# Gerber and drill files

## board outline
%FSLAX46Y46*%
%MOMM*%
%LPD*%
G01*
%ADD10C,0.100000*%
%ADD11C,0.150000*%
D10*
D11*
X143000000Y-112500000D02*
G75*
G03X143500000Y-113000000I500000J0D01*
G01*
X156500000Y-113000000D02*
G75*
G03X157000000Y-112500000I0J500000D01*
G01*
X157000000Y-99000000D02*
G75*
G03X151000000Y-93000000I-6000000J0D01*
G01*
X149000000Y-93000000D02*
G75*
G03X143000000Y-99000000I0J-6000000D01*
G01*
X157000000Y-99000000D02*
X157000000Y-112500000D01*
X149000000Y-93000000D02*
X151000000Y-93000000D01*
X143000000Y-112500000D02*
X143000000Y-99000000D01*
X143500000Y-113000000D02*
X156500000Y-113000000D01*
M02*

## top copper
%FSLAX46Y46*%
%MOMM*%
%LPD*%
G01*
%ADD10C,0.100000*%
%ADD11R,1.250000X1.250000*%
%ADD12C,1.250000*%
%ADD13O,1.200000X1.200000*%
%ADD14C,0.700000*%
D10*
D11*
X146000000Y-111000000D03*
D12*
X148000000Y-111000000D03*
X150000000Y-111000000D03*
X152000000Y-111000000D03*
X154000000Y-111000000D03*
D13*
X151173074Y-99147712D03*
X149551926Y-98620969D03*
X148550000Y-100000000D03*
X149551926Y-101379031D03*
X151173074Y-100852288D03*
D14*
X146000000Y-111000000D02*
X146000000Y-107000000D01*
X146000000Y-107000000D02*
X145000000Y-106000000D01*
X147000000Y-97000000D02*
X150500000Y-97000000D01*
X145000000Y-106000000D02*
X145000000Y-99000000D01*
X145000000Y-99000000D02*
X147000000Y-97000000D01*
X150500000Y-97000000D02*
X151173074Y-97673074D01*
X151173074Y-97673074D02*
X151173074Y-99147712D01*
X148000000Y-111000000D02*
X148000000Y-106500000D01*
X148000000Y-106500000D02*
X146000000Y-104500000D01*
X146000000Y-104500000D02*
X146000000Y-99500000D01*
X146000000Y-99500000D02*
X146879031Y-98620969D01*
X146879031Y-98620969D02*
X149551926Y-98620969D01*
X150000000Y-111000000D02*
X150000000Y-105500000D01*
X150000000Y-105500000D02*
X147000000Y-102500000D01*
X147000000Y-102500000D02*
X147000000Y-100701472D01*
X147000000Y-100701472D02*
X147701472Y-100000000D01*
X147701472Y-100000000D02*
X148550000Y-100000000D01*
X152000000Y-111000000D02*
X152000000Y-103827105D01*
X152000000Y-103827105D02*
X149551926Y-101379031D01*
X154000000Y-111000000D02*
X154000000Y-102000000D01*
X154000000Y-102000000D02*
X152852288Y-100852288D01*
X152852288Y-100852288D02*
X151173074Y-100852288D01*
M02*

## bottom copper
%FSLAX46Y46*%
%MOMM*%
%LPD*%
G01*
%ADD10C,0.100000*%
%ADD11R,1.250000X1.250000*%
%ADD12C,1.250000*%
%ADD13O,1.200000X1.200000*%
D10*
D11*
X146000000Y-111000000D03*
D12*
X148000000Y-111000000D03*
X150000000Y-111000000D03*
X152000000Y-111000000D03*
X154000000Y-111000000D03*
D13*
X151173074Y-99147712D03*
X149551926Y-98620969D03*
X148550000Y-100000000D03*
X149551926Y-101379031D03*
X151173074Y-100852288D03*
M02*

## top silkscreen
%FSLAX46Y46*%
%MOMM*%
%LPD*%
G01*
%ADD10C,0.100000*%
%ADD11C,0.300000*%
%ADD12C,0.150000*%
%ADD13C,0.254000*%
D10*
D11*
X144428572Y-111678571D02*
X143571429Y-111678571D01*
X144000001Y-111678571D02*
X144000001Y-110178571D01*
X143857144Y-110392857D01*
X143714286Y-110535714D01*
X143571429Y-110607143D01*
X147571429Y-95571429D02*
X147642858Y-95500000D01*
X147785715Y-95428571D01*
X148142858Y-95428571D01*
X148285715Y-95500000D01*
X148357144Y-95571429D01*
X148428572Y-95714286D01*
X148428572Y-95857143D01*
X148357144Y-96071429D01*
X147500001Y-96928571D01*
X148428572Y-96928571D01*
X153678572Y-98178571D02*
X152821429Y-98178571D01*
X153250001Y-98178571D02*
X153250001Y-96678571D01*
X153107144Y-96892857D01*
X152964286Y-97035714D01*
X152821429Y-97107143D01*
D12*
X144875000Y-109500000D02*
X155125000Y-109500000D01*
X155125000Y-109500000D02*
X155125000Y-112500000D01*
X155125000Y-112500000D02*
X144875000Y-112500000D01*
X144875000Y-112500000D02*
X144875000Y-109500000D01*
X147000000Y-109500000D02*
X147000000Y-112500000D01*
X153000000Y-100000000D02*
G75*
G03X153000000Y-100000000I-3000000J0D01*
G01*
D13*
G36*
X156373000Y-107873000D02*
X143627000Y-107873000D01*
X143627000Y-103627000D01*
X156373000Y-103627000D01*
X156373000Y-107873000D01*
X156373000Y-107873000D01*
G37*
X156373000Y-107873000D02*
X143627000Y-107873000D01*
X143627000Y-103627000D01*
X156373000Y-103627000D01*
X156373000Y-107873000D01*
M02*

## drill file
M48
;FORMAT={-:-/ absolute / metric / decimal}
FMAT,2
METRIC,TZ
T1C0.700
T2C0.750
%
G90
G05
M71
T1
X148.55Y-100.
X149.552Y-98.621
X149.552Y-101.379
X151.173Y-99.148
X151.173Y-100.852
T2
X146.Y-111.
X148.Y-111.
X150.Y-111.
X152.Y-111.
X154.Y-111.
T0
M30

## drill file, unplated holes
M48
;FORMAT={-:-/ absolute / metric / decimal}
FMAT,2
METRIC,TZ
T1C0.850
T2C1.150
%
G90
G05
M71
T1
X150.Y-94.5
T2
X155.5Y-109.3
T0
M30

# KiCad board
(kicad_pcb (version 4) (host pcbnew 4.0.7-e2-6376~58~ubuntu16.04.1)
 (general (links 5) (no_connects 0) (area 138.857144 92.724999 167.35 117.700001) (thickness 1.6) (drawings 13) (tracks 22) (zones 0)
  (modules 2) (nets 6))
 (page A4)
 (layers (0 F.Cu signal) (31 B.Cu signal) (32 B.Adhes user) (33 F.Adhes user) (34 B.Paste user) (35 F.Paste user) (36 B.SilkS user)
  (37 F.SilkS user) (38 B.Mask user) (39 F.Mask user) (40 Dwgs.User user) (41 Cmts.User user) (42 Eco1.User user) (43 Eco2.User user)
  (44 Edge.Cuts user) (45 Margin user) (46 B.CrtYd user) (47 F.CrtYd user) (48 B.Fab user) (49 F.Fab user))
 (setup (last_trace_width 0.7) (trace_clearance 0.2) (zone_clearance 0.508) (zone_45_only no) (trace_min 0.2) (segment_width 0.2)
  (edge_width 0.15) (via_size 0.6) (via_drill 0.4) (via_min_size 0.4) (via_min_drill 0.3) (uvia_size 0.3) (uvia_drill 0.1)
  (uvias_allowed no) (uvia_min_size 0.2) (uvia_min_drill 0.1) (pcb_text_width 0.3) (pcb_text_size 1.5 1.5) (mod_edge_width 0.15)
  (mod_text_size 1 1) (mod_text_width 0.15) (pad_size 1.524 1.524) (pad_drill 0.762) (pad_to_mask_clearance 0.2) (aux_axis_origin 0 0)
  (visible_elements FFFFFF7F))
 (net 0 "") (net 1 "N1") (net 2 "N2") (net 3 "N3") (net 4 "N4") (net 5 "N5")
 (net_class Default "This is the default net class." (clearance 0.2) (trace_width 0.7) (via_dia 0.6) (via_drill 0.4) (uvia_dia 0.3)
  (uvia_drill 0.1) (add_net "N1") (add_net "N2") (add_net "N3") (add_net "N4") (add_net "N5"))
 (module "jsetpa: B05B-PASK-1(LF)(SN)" (layer F.Cu) (at 150 111)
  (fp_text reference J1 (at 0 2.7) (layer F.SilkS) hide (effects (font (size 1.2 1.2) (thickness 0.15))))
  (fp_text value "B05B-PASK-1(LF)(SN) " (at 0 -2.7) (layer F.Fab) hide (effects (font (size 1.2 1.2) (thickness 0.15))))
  (fp_line (start -5.125 -1.5) (end 5.125 -1.5) (layer F.SilkS) (width 0.15))
  (fp_line (start 5.125 -1.5) (end 5.125 1.5) (layer F.SilkS) (width 0.15))
  (fp_line (start 5.125 1.5) (end -5.125 1.5) (layer F.SilkS) (width 0.15))
  (fp_line (start -5.125 1.5) (end -5.125 -1.5) (layer F.SilkS) (width 0.15))
  (fp_line (start -3 -1.5) (end -3 1.5) (layer F.SilkS) (width 0.15))
  (pad 1 thru_hole rect (at -4 0) (size 1.25 1.25) (drill 0.75) (layers *.Cu *.Mask) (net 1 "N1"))
  (pad 2 thru_hole circle (at -2 0) (size 1.25 1.25) (drill 0.75) (layers *.Cu *.Mask) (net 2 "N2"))
  (pad 3 thru_hole circle (at 0 0) (size 1.25 1.25) (drill 0.75) (layers *.Cu *.Mask) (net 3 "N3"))
  (pad 4 thru_hole circle (at 2 0) (size 1.25 1.25) (drill 0.75) (layers *.Cu *.Mask) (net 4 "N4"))
  (pad 5 thru_hole circle (at 4 0) (size 1.25 1.25) (drill 0.75) (layers *.Cu *.Mask) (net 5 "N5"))
  (pad "" np_thru_hole circle (at 5.5 -1.7) (size 1.15 1.15) (drill 1.15) (layers *.Cu *.Mask)))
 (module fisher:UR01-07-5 (layer F.Cu) (at 150 100)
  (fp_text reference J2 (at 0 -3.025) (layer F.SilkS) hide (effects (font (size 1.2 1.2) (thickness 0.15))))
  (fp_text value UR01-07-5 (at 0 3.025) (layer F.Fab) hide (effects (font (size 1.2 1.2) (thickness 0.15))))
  (fp_circle (center 0 0) (end 0 3) (layer F.SilkS) (width 0.15))
  (pad 1 thru_hole oval (at 1.173074 -0.852288) (size 1.2 1.2) (drill 0.7) (layers *.Cu *.Mask) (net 1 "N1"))
  (pad 2 thru_hole oval (at -0.448074 -1.379031) (size 1.2 1.2) (drill 0.7) (layers *.Cu *.Mask) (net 2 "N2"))
  (pad 3 thru_hole oval (at -1.45 0) (size 1.2 1.2) (drill 0.7) (layers *.Cu *.Mask) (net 3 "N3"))
  (pad 4 thru_hole oval (at -0.448074 1.379031) (size 1.2 1.2) (drill 0.7) (layers *.Cu *.Mask) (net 4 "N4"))
  (pad 5 thru_hole oval (at 1.173074 0.852288) (size 1.2 1.2) (drill 0.7) (layers *.Cu *.Mask) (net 5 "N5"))
  (pad "" np_thru_hole circle (at 0 -5.5) (size 0.85 0.85) (drill 0.85) (layers *.Cu *.Mask)))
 (gr_arc (start 143.5 112.5) (end 143.5 113) (angle 90) (layer Edge.Cuts) (width 0.15))
 (gr_arc (start 156.5 112.5) (end 157 112.5) (angle 90) (layer Edge.Cuts) (width 0.15))
 (gr_arc (start 151 99) (end 151 93) (angle 90) (layer Edge.Cuts) (width 0.15))
 (gr_arc (start 149 99) (end 143 99) (angle 90) (layer Edge.Cuts) (width 0.15))
 (gr_line (start 157 99) (end 157 112.5) (layer Edge.Cuts) (width 0.15))
 (gr_line (start 149 93) (end 151 93) (layer Edge.Cuts) (width 0.15))
 (gr_line (start 143 112.5) (end 143 99) (layer Edge.Cuts) (width 0.15))
 (gr_line (start 143.5 113) (end 156.5 113) (layer Edge.Cuts) (width 0.15))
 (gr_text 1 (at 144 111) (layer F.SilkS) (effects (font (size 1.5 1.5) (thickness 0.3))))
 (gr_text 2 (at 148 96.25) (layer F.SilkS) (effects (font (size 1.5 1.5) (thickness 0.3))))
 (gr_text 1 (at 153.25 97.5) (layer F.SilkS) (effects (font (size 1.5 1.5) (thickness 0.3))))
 (segment (start 146 111) (end 146 107) (width 0.7) (layer F.Cu) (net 1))
 (segment (start 146 107) (end 145 106) (width 0.7) (layer F.Cu) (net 1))
 (segment (start 147 97) (end 150.5 97) (width 0.7) (layer F.Cu) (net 1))
 (segment (start 145 106) (end 145 99) (width 0.7) (layer F.Cu) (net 1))
 (segment (start 145 99) (end 147 97) (width 0.7) (layer F.Cu) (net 1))
 (segment (start 150.5 97) (end 151.173074 97.673074) (width 0.7) (layer F.Cu) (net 1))
 (segment (start 151.173074 97.673074) (end 151.173074 99.147712) (width 0.7) (layer F.Cu) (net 1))
 (segment (start 148 111) (end 148 106.5) (width 0.7) (layer F.Cu) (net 2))
 (segment (start 148 106.5) (end 146 104.5) (width 0.7) (layer F.Cu) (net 2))
 (segment (start 146 104.5) (end 146 99.5) (width 0.7) (layer F.Cu) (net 2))
 (segment (start 146 99.5) (end 146.879031 98.620969) (width 0.7) (layer F.Cu) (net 2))
 (segment (start 146.879031 98.620969) (end 149.551926 98.620969) (width 0.7) (layer F.Cu) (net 2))
 (segment (start 150 111) (end 150 105.5) (width 0.7) (layer F.Cu) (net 3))
 (segment (start 150 105.5) (end 147 102.5) (width 0.7) (layer F.Cu) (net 3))
 (segment (start 147 102.5) (end 147 100.701472) (width 0.7) (layer F.Cu) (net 3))
 (segment (start 147 100.701472) (end 147.701472 100) (width 0.7) (layer F.Cu) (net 3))
 (segment (start 147.701472 100) (end 148.55 100) (width 0.7) (layer F.Cu) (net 3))
 (segment (start 152 111) (end 152 103.827105) (width 0.7) (layer F.Cu) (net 4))
 (segment (start 152 103.827105) (end 149.551926 101.379031) (width 0.7) (layer F.Cu) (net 4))
 (segment (start 154 111) (end 154 102) (width 0.7) (layer F.Cu) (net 5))
 (segment (start 154 102) (end 152.852288 100.852288) (width 0.7) (layer F.Cu) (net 5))
 (segment (start 152.852288 100.852288) (end 151.173074 100.852288) (width 0.7) (layer F.Cu) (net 5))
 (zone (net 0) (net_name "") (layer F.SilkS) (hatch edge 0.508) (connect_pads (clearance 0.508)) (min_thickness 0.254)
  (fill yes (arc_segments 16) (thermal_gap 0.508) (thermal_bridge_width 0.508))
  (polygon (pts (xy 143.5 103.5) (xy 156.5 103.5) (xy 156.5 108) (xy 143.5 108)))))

